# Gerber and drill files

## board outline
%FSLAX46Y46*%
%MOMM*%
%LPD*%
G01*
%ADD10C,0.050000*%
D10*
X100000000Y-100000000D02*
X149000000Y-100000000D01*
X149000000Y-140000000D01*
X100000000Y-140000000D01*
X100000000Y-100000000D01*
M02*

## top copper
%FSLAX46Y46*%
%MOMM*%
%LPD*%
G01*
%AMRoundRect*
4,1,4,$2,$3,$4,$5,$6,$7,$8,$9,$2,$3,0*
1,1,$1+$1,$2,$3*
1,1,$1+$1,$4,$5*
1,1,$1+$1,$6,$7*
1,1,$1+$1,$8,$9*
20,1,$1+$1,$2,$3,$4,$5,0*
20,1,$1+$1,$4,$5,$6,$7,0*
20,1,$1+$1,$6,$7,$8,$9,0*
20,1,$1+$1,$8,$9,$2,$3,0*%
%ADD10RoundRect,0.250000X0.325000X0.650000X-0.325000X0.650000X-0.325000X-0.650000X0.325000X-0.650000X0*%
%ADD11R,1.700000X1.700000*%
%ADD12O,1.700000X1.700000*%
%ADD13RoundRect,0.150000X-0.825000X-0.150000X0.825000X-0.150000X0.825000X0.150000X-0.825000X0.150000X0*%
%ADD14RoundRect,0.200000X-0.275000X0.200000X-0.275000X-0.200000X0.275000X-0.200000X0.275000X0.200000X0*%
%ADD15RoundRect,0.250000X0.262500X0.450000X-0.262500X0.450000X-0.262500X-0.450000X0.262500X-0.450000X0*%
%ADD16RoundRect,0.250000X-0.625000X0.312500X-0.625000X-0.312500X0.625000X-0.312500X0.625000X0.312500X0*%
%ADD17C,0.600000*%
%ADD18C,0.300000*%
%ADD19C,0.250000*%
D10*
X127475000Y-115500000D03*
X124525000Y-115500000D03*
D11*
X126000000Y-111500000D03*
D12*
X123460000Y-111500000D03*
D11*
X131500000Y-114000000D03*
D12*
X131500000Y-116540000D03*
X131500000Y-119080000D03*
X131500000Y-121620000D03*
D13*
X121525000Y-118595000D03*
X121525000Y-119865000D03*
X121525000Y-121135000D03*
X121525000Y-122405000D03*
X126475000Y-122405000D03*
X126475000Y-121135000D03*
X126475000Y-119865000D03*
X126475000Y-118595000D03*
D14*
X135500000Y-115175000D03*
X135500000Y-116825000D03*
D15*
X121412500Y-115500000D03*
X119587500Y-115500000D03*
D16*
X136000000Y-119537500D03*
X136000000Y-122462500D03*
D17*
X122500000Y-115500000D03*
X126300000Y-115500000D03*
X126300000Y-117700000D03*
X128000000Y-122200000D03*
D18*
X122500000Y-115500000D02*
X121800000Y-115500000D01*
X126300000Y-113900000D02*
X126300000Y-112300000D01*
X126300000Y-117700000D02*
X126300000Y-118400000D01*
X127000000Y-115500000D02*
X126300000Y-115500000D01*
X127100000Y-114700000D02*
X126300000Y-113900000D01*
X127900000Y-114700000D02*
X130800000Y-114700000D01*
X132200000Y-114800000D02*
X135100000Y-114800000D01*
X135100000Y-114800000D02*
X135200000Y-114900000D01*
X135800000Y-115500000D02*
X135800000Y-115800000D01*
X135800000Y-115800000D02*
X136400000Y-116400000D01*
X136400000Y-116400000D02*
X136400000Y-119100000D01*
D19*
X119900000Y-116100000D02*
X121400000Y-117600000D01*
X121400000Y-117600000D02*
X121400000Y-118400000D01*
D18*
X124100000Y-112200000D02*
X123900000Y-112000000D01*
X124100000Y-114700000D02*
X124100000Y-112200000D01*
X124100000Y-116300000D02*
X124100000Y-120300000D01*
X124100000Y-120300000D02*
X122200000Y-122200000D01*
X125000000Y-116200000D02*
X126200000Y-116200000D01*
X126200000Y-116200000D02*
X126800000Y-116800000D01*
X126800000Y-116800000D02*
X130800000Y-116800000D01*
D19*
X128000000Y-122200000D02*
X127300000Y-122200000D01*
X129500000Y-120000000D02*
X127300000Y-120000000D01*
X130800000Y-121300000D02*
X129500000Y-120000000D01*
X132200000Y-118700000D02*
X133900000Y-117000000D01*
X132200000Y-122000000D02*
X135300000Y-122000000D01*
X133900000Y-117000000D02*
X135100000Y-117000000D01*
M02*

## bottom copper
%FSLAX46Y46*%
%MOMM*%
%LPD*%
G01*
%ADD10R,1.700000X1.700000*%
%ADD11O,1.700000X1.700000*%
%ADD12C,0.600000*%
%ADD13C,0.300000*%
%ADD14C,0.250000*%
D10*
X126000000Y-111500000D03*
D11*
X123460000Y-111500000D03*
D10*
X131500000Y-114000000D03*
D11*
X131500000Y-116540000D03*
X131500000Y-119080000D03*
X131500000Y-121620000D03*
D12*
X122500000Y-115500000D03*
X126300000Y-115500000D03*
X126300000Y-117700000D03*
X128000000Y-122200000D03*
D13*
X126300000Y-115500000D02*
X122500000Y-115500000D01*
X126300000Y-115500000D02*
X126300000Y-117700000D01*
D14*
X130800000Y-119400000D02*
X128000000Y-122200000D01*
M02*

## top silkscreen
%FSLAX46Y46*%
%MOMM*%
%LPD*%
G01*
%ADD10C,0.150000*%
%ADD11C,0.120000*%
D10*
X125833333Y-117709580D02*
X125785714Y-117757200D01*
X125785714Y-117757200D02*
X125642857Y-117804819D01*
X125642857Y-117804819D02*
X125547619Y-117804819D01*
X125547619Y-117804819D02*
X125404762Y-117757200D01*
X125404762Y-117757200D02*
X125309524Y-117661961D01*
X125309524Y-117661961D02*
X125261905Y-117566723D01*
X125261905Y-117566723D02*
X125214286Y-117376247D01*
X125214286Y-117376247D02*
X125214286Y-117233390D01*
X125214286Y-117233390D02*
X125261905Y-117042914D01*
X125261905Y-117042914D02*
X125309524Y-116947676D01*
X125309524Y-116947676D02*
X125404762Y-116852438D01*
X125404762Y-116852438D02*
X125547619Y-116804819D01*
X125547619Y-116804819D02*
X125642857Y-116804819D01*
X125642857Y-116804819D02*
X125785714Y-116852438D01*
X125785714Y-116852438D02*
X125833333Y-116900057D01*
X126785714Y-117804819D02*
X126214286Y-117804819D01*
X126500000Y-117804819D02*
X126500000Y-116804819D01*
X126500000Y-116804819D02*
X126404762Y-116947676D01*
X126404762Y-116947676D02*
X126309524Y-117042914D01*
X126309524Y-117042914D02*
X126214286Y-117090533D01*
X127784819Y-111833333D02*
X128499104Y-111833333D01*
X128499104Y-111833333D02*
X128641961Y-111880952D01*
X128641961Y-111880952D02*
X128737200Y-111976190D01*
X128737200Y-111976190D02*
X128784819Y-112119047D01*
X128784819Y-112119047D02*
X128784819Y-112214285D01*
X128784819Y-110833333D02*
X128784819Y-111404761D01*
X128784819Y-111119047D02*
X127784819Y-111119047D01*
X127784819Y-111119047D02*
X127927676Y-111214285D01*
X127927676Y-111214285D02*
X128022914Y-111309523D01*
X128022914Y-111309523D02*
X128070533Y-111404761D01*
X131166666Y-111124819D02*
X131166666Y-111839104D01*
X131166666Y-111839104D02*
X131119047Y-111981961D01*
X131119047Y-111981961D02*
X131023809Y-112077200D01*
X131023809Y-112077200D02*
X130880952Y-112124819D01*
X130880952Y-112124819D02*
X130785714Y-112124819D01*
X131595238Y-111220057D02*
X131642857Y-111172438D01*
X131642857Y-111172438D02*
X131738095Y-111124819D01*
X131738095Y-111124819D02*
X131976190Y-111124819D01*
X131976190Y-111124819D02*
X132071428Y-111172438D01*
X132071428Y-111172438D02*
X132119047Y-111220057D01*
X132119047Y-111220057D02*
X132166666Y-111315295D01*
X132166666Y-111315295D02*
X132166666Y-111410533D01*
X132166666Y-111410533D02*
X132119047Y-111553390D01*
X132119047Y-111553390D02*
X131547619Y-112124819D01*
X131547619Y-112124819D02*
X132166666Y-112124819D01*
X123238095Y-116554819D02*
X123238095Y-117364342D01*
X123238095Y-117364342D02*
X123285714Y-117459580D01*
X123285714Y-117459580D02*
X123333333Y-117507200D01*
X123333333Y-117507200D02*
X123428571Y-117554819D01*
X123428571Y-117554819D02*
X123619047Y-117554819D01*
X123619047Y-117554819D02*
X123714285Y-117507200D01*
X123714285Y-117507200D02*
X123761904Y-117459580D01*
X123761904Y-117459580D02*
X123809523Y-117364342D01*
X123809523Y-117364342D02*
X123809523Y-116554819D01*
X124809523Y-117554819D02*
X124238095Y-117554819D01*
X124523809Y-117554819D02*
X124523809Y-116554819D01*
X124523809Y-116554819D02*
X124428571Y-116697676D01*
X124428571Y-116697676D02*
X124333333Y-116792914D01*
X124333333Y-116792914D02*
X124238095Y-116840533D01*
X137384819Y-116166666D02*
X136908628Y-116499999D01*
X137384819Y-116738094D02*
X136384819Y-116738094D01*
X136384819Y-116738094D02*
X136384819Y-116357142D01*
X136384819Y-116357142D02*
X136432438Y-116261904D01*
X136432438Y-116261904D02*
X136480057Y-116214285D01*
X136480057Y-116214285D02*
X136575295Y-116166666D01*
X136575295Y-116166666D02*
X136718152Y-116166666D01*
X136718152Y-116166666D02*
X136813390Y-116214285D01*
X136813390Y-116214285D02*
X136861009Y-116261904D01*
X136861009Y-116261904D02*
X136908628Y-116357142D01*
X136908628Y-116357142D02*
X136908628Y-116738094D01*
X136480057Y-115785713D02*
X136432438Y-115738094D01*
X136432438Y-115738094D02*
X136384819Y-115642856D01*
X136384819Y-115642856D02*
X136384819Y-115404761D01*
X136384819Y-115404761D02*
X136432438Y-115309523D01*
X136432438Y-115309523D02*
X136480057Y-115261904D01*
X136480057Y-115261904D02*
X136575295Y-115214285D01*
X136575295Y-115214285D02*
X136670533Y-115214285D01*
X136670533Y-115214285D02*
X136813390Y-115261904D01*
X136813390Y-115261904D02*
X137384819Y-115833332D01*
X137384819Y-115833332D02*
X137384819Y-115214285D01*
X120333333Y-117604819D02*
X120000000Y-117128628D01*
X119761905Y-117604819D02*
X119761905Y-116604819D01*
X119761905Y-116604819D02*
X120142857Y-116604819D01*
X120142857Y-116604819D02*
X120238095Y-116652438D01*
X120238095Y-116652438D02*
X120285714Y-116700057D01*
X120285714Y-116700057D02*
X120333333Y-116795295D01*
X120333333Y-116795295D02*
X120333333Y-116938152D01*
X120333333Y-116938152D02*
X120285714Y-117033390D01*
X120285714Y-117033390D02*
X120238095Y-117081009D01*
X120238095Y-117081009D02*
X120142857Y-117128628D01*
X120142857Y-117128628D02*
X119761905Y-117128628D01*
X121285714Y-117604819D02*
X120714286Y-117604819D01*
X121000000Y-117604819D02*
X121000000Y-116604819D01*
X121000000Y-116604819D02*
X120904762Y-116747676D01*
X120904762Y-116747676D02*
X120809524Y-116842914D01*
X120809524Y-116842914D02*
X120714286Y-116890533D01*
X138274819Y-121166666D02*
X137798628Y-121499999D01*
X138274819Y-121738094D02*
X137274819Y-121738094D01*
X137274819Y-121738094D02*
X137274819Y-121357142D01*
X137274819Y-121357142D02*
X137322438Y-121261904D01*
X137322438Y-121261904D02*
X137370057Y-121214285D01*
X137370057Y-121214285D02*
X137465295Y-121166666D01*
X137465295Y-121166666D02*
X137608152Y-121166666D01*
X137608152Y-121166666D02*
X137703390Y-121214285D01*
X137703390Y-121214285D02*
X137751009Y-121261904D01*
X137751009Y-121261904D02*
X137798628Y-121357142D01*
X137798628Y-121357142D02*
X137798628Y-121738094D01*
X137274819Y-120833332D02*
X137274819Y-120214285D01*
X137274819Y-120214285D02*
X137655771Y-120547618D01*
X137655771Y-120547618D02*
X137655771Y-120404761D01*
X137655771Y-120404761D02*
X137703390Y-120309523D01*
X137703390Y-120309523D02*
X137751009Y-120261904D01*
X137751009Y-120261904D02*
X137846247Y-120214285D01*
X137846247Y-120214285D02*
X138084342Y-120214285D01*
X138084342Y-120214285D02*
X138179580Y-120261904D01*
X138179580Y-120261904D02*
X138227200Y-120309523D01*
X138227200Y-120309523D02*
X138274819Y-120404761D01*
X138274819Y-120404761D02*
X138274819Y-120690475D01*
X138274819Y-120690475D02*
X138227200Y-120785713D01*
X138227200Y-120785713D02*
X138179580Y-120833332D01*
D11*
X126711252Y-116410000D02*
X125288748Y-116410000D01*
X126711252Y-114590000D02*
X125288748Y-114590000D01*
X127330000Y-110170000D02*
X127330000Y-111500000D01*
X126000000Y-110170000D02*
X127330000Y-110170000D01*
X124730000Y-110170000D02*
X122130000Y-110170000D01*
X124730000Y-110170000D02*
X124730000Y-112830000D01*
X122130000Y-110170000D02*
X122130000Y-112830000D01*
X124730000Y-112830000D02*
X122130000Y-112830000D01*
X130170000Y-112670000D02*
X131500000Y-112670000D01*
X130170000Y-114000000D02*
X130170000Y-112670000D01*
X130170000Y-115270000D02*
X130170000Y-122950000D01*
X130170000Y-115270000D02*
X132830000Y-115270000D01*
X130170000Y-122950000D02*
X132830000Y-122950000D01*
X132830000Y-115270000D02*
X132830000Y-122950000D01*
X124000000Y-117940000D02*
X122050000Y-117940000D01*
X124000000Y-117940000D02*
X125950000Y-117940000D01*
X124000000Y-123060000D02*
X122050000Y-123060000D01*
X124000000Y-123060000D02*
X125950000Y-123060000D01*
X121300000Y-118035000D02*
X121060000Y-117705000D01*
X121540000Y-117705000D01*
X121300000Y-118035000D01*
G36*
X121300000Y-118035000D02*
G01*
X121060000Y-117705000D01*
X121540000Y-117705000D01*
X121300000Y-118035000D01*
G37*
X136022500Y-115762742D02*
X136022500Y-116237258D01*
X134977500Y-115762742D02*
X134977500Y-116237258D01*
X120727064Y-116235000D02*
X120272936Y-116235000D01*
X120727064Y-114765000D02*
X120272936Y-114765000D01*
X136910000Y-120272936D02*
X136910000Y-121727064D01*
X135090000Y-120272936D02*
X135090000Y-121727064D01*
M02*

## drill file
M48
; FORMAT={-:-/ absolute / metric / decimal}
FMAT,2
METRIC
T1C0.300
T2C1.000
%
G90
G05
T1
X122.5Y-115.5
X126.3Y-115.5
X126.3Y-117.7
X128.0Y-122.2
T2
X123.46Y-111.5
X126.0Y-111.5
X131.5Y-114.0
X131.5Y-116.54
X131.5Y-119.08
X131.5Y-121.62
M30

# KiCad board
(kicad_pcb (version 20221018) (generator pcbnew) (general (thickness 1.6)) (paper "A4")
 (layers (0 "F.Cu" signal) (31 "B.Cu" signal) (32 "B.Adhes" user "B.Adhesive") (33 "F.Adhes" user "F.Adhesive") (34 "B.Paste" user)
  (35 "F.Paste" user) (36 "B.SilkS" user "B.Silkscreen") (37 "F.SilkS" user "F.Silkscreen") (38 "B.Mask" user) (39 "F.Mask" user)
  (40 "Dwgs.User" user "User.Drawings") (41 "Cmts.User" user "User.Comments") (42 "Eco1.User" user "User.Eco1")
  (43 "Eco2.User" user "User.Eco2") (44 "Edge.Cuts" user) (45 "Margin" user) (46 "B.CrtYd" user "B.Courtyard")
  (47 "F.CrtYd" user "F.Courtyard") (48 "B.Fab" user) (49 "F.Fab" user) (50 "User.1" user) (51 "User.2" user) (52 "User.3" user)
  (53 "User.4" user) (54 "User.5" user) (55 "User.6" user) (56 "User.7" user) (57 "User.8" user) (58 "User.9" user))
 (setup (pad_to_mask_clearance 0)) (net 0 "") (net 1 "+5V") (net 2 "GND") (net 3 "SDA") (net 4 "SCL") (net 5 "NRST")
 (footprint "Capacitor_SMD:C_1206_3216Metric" (layer "F.Cu") (at 126 115.5 180)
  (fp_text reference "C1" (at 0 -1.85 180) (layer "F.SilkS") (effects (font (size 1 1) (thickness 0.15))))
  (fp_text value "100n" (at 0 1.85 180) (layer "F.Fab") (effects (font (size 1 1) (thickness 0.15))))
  (fp_line (start -0.711252 -0.91) (end 0.711252 -0.91) (stroke (width 0.12) (type solid)) (layer "F.SilkS"))
  (fp_line (start -0.711252 0.91) (end 0.711252 0.91) (stroke (width 0.12) (type solid)) (layer "F.SilkS"))
  (pad "1" smd roundrect (at -1.475 0 180) (size 1.15 1.8) (layers "F.Cu" "F.Paste" "F.Mask") (roundrect_rratio 0.217391) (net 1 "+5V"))
  (pad "2" smd roundrect (at 1.475 0 180) (size 1.15 1.8) (layers "F.Cu" "F.Paste" "F.Mask") (roundrect_rratio 0.217391) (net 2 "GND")))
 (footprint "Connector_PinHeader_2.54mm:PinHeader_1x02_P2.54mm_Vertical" (layer "F.Cu") (at 126 111.5 -90)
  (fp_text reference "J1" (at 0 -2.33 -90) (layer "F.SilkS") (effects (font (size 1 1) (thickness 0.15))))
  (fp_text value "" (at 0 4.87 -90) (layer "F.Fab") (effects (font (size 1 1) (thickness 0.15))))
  (fp_line (start -1.33 -1.33) (end 0 -1.33) (stroke (width 0.12) (type solid)) (layer "F.SilkS"))
  (fp_line (start -1.33 0) (end -1.33 -1.33) (stroke (width 0.12) (type solid)) (layer "F.SilkS"))
  (fp_line (start -1.33 1.27) (end -1.33 3.87) (stroke (width 0.12) (type solid)) (layer "F.SilkS"))
  (fp_line (start -1.33 1.27) (end 1.33 1.27) (stroke (width 0.12) (type solid)) (layer "F.SilkS"))
  (fp_line (start -1.33 3.87) (end 1.33 3.87) (stroke (width 0.12) (type solid)) (layer "F.SilkS"))
  (fp_line (start 1.33 1.27) (end 1.33 3.87) (stroke (width 0.12) (type solid)) (layer "F.SilkS"))
  (pad "1" thru_hole rect (at 0 0 270) (size 1.7 1.7) (drill 1) (layers "*.Cu" "*.Mask") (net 1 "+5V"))
  (pad "2" thru_hole oval (at 0 2.54 270) (size 1.7 1.7) (drill 1) (layers "*.Cu" "*.Mask") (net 2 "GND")))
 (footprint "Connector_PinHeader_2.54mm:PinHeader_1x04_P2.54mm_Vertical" (layer "F.Cu") (at 131.5 114)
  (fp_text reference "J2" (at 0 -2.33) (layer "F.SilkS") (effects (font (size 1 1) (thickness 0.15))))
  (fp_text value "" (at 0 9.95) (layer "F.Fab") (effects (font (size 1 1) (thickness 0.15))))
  (fp_line (start -1.33 -1.33) (end 0 -1.33) (stroke (width 0.12) (type solid)) (layer "F.SilkS"))
  (fp_line (start -1.33 0) (end -1.33 -1.33) (stroke (width 0.12) (type solid)) (layer "F.SilkS"))
  (fp_line (start -1.33 1.27) (end -1.33 8.95) (stroke (width 0.12) (type solid)) (layer "F.SilkS"))
  (fp_line (start -1.33 1.27) (end 1.33 1.27) (stroke (width 0.12) (type solid)) (layer "F.SilkS"))
  (fp_line (start -1.33 8.95) (end 1.33 8.95) (stroke (width 0.12) (type solid)) (layer "F.SilkS"))
  (fp_line (start 1.33 1.27) (end 1.33 8.95) (stroke (width 0.12) (type solid)) (layer "F.SilkS"))
  (pad "1" thru_hole rect (at 0 0) (size 1.7 1.7) (drill 1) (layers "*.Cu" "*.Mask") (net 1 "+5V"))
  (pad "2" thru_hole oval (at 0 2.54) (size 1.7 1.7) (drill 1) (layers "*.Cu" "*.Mask") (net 2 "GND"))
  (pad "3" thru_hole oval (at 0 5.08) (size 1.7 1.7) (drill 1) (layers "*.Cu" "*.Mask") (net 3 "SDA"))
  (pad "4" thru_hole oval (at 0 7.62) (size 1.7 1.7) (drill 1) (layers "*.Cu" "*.Mask") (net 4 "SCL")))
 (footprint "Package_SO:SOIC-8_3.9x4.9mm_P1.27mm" (layer "F.Cu") (at 124 120.5)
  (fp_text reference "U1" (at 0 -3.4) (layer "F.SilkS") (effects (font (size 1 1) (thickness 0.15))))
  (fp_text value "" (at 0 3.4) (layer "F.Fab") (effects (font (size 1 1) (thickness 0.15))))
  (fp_line (start 0 -2.56) (end -1.95 -2.56) (stroke (width 0.12) (type solid)) (layer "F.SilkS"))
  (fp_line (start 0 -2.56) (end 1.95 -2.56) (stroke (width 0.12) (type solid)) (layer "F.SilkS"))
  (fp_line (start 0 2.56) (end -1.95 2.56) (stroke (width 0.12) (type solid)) (layer "F.SilkS"))
  (fp_line (start 0 2.56) (end 1.95 2.56) (stroke (width 0.12) (type solid)) (layer "F.SilkS"))
  (fp_poly
   (pts (xy -2.7 -2.465) (xy -2.94 -2.795) (xy -2.46 -2.795) (xy -2.7 -2.465)) (stroke (width 0.12) (type solid)) (fill solid)
   (layer "F.SilkS"))
  (pad "1" smd roundrect (at -2.475 -1.905) (size 1.95 0.6) (layers "F.Cu" "F.Paste" "F.Mask") (roundrect_rratio 0.25) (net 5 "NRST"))
  (pad "2" smd roundrect (at -2.475 -0.635) (size 1.95 0.6) (layers "F.Cu" "F.Paste" "F.Mask") (roundrect_rratio 0.25))
  (pad "3" smd roundrect (at -2.475 0.635) (size 1.95 0.6) (layers "F.Cu" "F.Paste" "F.Mask") (roundrect_rratio 0.25))
  (pad "4" smd roundrect (at -2.475 1.905) (size 1.95 0.6) (layers "F.Cu" "F.Paste" "F.Mask") (roundrect_rratio 0.25) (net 2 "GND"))
  (pad "5" smd roundrect (at 2.475 1.905) (size 1.95 0.6) (layers "F.Cu" "F.Paste" "F.Mask") (roundrect_rratio 0.25) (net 3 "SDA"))
  (pad "6" smd roundrect (at 2.475 0.635) (size 1.95 0.6) (layers "F.Cu" "F.Paste" "F.Mask") (roundrect_rratio 0.25))
  (pad "7" smd roundrect (at 2.475 -0.635) (size 1.95 0.6) (layers "F.Cu" "F.Paste" "F.Mask") (roundrect_rratio 0.25) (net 4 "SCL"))
  (pad "8" smd roundrect (at 2.475 -1.905) (size 1.95 0.6) (layers "F.Cu" "F.Paste" "F.Mask") (roundrect_rratio 0.25) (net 1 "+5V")))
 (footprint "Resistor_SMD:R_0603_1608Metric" (layer "F.Cu") (at 135.5 116 -90)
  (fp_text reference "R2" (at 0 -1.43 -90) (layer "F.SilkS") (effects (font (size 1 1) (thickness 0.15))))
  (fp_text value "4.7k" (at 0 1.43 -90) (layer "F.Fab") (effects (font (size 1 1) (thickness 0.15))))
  (fp_line (start -0.237258 -0.5225) (end 0.237258 -0.5225) (stroke (width 0.12) (type solid)) (layer "F.SilkS"))
  (fp_line (start -0.237258 0.5225) (end 0.237258 0.5225) (stroke (width 0.12) (type solid)) (layer "F.SilkS"))
  (pad "1" smd roundrect (at -0.825 0 270) (size 0.8 0.95) (layers "F.Cu" "F.Paste" "F.Mask") (roundrect_rratio 0.25) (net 1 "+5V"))
  (pad "2" smd roundrect (at 0.825 0 270) (size 0.8 0.95) (layers "F.Cu" "F.Paste" "F.Mask") (roundrect_rratio 0.25) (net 3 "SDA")))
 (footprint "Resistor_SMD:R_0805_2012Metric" (layer "F.Cu") (at 120.5 115.5 180)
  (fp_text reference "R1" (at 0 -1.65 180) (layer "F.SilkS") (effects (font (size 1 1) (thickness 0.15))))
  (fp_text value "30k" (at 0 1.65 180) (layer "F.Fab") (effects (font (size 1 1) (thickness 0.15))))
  (fp_line (start -0.227064 -0.735) (end 0.227064 -0.735) (stroke (width 0.12) (type solid)) (layer "F.SilkS"))
  (fp_line (start -0.227064 0.735) (end 0.227064 0.735) (stroke (width 0.12) (type solid)) (layer "F.SilkS"))
  (pad "1" smd roundrect (at -0.9125 0 180) (size 1.025 1.4) (layers "F.Cu" "F.Paste" "F.Mask") (roundrect_rratio 0.243902) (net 1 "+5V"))
  (pad "2" smd roundrect (at 0.9125 0 180) (size 1.025 1.4) (layers "F.Cu" "F.Paste" "F.Mask") (roundrect_rratio 0.243902) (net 5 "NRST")))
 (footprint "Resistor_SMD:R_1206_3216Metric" (layer "F.Cu") (at 136 121 -90)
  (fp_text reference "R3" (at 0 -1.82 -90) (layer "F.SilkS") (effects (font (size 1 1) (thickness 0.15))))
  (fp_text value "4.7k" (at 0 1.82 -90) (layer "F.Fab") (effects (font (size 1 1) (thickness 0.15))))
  (fp_line (start -0.727064 -0.91) (end 0.727064 -0.91) (stroke (width 0.12) (type solid)) (layer "F.SilkS"))
  (fp_line (start -0.727064 0.91) (end 0.727064 0.91) (stroke (width 0.12) (type solid)) (layer "F.SilkS"))
  (pad "1" smd roundrect (at -1.4625 0 270) (size 1.125 1.75) (layers "F.Cu" "F.Paste" "F.Mask") (roundrect_rratio 0.222222) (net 1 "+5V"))
  (pad "2" smd roundrect (at 1.4625 0 270) (size 1.125 1.75) (layers "F.Cu" "F.Paste" "F.Mask") (roundrect_rratio 0.222222) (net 4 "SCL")))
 (gr_rect (start 100 100) (end 149 140) (stroke (width 0.05) (type default)) (fill none) (layer "Edge.Cuts"))
 (segment (start 122.5 115.5) (end 121.8 115.5) (width 0.3) (layer "F.Cu") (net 1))
 (segment (start 126.3 113.9) (end 126.3 112.3) (width 0.3) (layer "F.Cu") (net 1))
 (segment (start 126.3 117.7) (end 126.3 118.4) (width 0.3) (layer "F.Cu") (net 1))
 (segment (start 127 115.5) (end 126.3 115.5) (width 0.3) (layer "F.Cu") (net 1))
 (segment (start 127.1 114.7) (end 126.3 113.9) (width 0.3) (layer "F.Cu") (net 1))
 (segment (start 127.9 114.7) (end 130.8 114.7) (width 0.3) (layer "F.Cu") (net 1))
 (segment (start 132.2 114.8) (end 135.1 114.8) (width 0.3) (layer "F.Cu") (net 1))
 (segment (start 135.1 114.8) (end 135.2 114.9) (width 0.3) (layer "F.Cu") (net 1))
 (segment (start 135.8 115.5) (end 135.8 115.8) (width 0.3) (layer "F.Cu") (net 1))
 (segment (start 135.8 115.8) (end 136.4 116.4) (width 0.3) (layer "F.Cu") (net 1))
 (segment (start 136.4 116.4) (end 136.4 119.1) (width 0.3) (layer "F.Cu") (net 1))
 (via (at 122.5 115.5) (size 0.6) (drill 0.3) (layers "F.Cu" "B.Cu") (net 1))
 (via (at 126.3 115.5) (size 0.6) (drill 0.3) (layers "F.Cu" "B.Cu") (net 1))
 (via (at 126.3 117.7) (size 0.6) (drill 0.3) (layers "F.Cu" "B.Cu") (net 1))
 (segment (start 119.9 116.1) (end 121.4 117.6) (width 0.25) (layer "F.Cu") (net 5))
 (segment (start 121.4 117.6) (end 121.4 118.4) (width 0.25) (layer "F.Cu") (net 5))
 (segment (start 124.1 112.2) (end 123.9 112) (width 0.3) (layer "F.Cu") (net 2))
 (segment (start 124.1 114.7) (end 124.1 112.2) (width 0.3) (layer "F.Cu") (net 2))
 (segment (start 124.1 116.3) (end 124.1 120.3) (width 0.3) (layer "F.Cu") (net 2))
 (segment (start 124.1 120.3) (end 122.2 122.2) (width 0.3) (layer "F.Cu") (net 2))
 (segment (start 125 116.2) (end 126.2 116.2) (width 0.3) (layer "F.Cu") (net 2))
 (segment (start 126.2 116.2) (end 126.8 116.8) (width 0.3) (layer "F.Cu") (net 2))
 (segment (start 126.3 115.5) (end 122.5 115.5) (width 0.3) (layer "B.Cu") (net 1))
 (segment (start 126.3 115.5) (end 126.3 117.7) (width 0.3) (layer "B.Cu") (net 1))
 (segment (start 126.8 116.8) (end 130.8 116.8) (width 0.3) (layer "F.Cu") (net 2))
 (segment (start 128 122.2) (end 127.3 122.2) (width 0.25) (layer "F.Cu") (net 3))
 (segment (start 129.5 120) (end 127.3 120) (width 0.25) (layer "F.Cu") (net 4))
 (segment (start 130.8 121.3) (end 129.5 120) (width 0.25) (layer "F.Cu") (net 4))
 (segment (start 132.2 118.7) (end 133.9 117) (width 0.25) (layer "F.Cu") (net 3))
 (segment (start 132.2 122) (end 135.3 122) (width 0.25) (layer "F.Cu") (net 4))
 (segment (start 133.9 117) (end 135.1 117) (width 0.25) (layer "F.Cu") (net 3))
 (via (at 128 122.2) (size 0.6) (drill 0.3) (layers "F.Cu" "B.Cu") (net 3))
 (segment (start 130.8 119.4) (end 128 122.2) (width 0.25) (layer "B.Cu") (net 3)))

